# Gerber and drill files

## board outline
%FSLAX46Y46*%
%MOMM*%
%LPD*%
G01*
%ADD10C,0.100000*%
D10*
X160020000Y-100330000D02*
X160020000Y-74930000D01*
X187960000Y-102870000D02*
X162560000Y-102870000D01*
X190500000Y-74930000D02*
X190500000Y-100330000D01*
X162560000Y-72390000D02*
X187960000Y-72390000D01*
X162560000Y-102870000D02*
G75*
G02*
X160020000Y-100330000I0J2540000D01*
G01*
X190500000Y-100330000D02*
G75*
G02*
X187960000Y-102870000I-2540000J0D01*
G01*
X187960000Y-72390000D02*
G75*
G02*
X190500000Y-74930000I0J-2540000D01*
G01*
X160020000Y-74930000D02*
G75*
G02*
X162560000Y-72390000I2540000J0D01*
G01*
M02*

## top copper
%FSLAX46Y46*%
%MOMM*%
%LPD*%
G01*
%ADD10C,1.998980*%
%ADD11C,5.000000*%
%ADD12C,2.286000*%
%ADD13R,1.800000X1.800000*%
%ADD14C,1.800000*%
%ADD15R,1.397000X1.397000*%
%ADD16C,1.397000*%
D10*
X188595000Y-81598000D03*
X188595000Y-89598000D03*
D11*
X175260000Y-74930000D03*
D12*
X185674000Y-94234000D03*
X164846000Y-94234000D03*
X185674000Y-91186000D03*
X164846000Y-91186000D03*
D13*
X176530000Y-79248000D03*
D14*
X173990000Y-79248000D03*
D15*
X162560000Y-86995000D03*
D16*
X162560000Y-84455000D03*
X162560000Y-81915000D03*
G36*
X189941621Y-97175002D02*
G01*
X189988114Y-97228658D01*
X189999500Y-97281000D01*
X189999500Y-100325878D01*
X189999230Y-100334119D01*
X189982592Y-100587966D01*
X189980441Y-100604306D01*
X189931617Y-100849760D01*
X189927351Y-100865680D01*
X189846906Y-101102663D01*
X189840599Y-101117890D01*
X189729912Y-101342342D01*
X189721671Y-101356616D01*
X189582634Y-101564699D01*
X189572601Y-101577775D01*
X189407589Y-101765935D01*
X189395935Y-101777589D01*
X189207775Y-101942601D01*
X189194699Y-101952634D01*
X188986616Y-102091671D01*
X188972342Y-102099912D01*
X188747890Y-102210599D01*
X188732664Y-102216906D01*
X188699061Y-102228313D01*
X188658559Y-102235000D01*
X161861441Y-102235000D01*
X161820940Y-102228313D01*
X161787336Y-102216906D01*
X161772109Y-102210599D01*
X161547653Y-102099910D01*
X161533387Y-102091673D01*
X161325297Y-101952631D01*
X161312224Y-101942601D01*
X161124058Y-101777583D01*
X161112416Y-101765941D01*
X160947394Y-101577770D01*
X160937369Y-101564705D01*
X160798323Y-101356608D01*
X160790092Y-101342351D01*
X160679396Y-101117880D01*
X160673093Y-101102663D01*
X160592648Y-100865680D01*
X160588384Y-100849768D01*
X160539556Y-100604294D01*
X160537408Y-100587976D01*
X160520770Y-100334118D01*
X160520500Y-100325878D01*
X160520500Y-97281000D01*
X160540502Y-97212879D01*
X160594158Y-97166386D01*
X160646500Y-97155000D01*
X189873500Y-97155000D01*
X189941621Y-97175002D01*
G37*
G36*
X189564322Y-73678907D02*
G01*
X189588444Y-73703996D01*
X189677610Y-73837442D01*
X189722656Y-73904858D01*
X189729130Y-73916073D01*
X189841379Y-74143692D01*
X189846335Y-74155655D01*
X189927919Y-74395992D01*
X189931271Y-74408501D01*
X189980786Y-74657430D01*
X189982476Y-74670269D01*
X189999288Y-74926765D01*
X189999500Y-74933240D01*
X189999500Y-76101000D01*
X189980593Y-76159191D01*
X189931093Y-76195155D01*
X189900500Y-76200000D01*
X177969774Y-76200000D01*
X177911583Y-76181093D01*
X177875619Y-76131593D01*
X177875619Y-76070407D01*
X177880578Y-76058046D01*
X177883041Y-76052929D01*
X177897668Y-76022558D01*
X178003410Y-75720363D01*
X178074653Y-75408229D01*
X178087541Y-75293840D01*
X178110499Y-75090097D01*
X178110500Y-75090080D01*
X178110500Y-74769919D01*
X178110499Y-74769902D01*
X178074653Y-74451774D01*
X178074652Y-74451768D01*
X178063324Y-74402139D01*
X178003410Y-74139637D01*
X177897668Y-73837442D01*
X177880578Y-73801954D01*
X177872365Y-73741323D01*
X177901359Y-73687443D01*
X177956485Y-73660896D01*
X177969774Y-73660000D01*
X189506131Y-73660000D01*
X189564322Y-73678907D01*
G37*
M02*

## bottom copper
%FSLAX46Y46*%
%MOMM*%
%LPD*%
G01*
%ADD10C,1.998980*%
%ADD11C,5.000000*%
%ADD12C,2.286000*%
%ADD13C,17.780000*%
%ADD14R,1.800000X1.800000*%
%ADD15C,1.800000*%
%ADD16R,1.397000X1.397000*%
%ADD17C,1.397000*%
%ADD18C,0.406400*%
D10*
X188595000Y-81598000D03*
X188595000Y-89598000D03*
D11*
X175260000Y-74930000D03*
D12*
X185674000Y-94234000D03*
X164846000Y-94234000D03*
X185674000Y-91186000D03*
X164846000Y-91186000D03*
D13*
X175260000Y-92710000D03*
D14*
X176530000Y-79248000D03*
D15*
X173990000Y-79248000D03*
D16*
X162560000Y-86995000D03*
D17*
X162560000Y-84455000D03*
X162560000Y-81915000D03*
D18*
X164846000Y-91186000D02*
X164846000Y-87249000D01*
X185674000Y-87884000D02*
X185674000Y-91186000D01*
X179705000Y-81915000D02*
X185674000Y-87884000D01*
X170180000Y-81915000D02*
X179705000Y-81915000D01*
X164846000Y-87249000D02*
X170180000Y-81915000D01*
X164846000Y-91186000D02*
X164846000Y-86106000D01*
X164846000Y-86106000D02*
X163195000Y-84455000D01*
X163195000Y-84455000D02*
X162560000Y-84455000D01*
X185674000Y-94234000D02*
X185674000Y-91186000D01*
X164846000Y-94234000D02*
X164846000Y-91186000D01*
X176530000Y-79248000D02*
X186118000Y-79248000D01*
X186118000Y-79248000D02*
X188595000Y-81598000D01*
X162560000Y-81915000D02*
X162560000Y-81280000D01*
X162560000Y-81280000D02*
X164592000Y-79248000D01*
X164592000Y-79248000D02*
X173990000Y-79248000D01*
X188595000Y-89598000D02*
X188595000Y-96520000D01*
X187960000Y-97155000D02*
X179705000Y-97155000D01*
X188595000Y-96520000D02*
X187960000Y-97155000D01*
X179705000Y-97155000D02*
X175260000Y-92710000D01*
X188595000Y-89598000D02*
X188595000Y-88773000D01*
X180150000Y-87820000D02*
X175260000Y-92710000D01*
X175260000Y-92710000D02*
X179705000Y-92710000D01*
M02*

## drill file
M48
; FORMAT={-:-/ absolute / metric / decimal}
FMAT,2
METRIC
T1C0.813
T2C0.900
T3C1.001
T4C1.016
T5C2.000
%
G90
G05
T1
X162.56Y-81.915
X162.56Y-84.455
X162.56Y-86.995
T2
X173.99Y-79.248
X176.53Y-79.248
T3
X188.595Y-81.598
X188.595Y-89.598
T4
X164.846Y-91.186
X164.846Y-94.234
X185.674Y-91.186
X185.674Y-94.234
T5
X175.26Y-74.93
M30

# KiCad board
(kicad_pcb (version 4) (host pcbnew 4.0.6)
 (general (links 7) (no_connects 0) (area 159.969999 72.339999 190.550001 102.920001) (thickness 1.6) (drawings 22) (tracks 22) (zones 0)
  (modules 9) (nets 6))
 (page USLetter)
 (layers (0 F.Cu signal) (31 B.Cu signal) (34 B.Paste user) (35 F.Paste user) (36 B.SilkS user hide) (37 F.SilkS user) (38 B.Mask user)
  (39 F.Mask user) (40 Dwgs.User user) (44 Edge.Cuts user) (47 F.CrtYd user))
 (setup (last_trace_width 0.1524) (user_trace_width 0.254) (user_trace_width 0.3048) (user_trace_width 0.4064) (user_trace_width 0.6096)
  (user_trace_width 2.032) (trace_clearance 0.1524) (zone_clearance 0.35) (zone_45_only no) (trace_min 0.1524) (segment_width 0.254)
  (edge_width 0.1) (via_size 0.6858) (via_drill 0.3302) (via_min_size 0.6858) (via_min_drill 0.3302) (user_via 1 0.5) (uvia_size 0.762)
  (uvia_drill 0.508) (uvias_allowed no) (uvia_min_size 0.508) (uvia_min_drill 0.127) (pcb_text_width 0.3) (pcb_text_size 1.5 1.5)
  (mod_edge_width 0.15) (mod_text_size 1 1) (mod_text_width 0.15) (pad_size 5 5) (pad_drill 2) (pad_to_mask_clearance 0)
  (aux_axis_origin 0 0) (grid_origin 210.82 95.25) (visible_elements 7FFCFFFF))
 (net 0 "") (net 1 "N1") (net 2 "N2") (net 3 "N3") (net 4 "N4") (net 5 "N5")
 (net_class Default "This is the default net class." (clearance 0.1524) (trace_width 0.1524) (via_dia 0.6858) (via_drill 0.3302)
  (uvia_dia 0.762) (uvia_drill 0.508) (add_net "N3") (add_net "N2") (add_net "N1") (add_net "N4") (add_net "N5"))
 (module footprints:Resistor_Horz (layer F.Cu) (at 188.595 85.598 270)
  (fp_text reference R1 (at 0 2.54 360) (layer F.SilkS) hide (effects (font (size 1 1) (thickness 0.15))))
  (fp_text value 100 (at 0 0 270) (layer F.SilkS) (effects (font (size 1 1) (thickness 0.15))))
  (pad 1 thru_hole circle (at -4 0 270) (size 1.99898 1.99898) (drill 1.00076) (layers *.Cu *.SilkS *.Mask) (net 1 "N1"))
  (pad 2 thru_hole circle (at 4 0 270) (size 1.99898 1.99898) (drill 1.00076) (layers *.Cu *.SilkS *.Mask) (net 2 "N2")))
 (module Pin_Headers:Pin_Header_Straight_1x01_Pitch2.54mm (layer F.Cu) (at 175.26 74.93)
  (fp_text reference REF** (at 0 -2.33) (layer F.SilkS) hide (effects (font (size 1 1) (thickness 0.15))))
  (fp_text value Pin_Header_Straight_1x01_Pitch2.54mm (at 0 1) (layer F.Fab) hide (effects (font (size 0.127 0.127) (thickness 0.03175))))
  (pad 1 thru_hole circle (at 0 0) (size 5 5) (drill 2) (layers *.Cu B.Mask)))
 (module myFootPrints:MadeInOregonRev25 (layer F.Cu) (at 167.64 76.454)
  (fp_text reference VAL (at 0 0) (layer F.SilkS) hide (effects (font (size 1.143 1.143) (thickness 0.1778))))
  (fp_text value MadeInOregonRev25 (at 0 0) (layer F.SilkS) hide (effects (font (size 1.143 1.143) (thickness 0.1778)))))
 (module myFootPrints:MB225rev (layer F.Cu) (at 184.15 76.2)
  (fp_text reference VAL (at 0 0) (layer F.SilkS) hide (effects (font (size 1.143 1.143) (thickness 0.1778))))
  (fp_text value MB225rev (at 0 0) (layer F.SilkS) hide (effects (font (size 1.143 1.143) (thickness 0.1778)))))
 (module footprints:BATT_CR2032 (layer B.Cu) (at 175.26 92.71 180)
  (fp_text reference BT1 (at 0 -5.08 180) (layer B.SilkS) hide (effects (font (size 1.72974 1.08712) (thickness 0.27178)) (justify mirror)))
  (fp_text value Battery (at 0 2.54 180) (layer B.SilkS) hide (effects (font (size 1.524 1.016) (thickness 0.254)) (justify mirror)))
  (pad 1 thru_hole circle (at -10.414 -1.524 180) (size 2.286 2.286) (drill 1.016) (layers *.Cu *.Mask B.SilkS) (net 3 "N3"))
  (pad 1 thru_hole circle (at 10.414 -1.524 180) (size 2.286 2.286) (drill 1.016) (layers *.Cu *.Mask B.SilkS) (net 3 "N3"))
  (pad 1 thru_hole circle (at -10.414 1.524 180) (size 2.286 2.286) (drill 1.016) (layers *.Cu *.Mask B.SilkS) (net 3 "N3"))
  (pad 1 thru_hole circle (at 10.414 1.524 180) (size 2.286 2.286) (drill 1.016) (layers *.Cu *.Mask B.SilkS) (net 3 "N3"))
  (pad 2 smd circle (at 0 0 180) (size 17.78 17.78) (layers B.Cu B.Paste B.Mask) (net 2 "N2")))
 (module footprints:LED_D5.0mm (layer F.Cu) (at 176.53 79.248 180)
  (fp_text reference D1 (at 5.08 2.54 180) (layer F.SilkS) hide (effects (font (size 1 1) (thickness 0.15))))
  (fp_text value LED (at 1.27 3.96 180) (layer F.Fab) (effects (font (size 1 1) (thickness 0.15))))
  (pad 1 thru_hole rect (at 0 0 180) (size 1.8 1.8) (drill 0.9) (layers *.Cu *.Mask) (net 1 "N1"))
  (pad 2 thru_hole circle (at 2.54 0 180) (size 1.8 1.8) (drill 0.9) (layers *.Cu *.Mask) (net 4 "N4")))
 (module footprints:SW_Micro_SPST (layer F.Cu) (at 162.56 84.455 90)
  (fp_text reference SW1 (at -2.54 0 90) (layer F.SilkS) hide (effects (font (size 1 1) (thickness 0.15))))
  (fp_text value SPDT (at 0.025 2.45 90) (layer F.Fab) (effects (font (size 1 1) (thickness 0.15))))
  (pad 1 thru_hole rect (at -2.54 0 90) (size 1.397 1.397) (drill 0.8128) (layers *.Cu *.Mask F.SilkS) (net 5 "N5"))
  (pad 2 thru_hole circle (at 0 0 90) (size 1.397 1.397) (drill 0.8128) (layers *.Cu *.Mask F.SilkS) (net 3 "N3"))
  (pad 3 thru_hole circle (at 2.54 0 90) (size 1.397 1.397) (drill 0.8128) (layers *.Cu *.Mask F.SilkS) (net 4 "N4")))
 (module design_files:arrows (layer F.Cu) (at 179.07 77.47)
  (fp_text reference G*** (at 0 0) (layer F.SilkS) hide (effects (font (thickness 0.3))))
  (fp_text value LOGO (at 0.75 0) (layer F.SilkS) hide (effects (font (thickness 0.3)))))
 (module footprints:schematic (layer F.Cu) (at 175.26 87.503)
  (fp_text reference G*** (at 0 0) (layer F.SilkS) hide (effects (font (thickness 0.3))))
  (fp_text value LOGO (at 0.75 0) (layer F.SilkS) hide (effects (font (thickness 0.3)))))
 (gr_line (start 160.02 100.33) (end 160.02 74.93) (angle 90) (layer Edge.Cuts) (width 0.1))
 (gr_line (start 187.96 102.87) (end 162.56 102.87) (angle 90) (layer Edge.Cuts) (width 0.1))
 (gr_line (start 190.5 74.93) (end 190.5 100.33) (angle 90) (layer Edge.Cuts) (width 0.1))
 (gr_line (start 162.56 72.39) (end 187.96 72.39) (angle 90) (layer Edge.Cuts) (width 0.1))
 (gr_arc (start 162.56 100.33) (end 162.56 102.87) (angle 90) (layer Edge.Cuts) (width 0.1))
 (gr_arc (start 187.96 100.33) (end 190.5 100.33) (angle 90) (layer Edge.Cuts) (width 0.1))
 (gr_arc (start 187.96 74.93) (end 187.96 72.39) (angle 90) (layer Edge.Cuts) (width 0.1))
 (gr_arc (start 162.56 74.93) (end 160.02 74.93) (angle 90) (layer Edge.Cuts) (width 0.1))
 (segment (start 164.846 91.186) (end 164.846 87.249) (width 0.4064) (layer B.Cu) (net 3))
 (segment (start 185.674 87.884) (end 185.674 91.186) (width 0.4064) (layer B.Cu) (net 3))
 (segment (start 179.705 81.915) (end 185.674 87.884) (width 0.4064) (layer B.Cu) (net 3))
 (segment (start 170.18 81.915) (end 179.705 81.915) (width 0.4064) (layer B.Cu) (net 3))
 (segment (start 164.846 87.249) (end 170.18 81.915) (width 0.4064) (layer B.Cu) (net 3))
 (segment (start 164.846 91.186) (end 164.846 86.106) (width 0.4064) (layer B.Cu) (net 3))
 (segment (start 164.846 86.106) (end 163.195 84.455) (width 0.4064) (layer B.Cu) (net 3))
 (segment (start 163.195 84.455) (end 162.56 84.455) (width 0.4064) (layer B.Cu) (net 3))
 (segment (start 185.674 94.234) (end 185.674 91.186) (width 0.4064) (layer B.Cu) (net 3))
 (segment (start 164.846 94.234) (end 164.846 91.186) (width 0.4064) (layer B.Cu) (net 3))
 (segment (start 176.53 79.248) (end 186.118 79.248) (width 0.4064) (layer B.Cu) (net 1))
 (segment (start 186.118 79.248) (end 188.595 81.598) (width 0.4064) (layer B.Cu) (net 1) (status 20))
 (segment (start 162.56 81.915) (end 162.56 81.28) (width 0.4064) (layer B.Cu) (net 4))
 (segment (start 162.56 81.28) (end 164.592 79.248) (width 0.4064) (layer B.Cu) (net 4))
 (segment (start 164.592 79.248) (end 173.99 79.248) (width 0.4064) (layer B.Cu) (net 4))
 (segment (start 188.595 89.598) (end 188.595 96.52) (width 0.4064) (layer B.Cu) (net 2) (status 10))
 (segment (start 187.96 97.155) (end 179.705 97.155) (width 0.4064) (layer B.Cu) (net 2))
 (segment (start 188.595 96.52) (end 187.96 97.155) (width 0.4064) (layer B.Cu) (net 2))
 (segment (start 179.705 97.155) (end 175.26 92.71) (width 0.4064) (layer B.Cu) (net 2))
 (segment (start 188.595 89.598) (end 188.595 88.773) (width 0.4064) (layer B.Cu) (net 2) (status 30))
 (segment (start 180.15 87.82) (end 175.26 92.71) (width 0.4064) (layer B.Cu) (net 2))
 (segment (start 175.26 92.71) (end 179.705 92.71) (width 0.4064) (layer B.Cu) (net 2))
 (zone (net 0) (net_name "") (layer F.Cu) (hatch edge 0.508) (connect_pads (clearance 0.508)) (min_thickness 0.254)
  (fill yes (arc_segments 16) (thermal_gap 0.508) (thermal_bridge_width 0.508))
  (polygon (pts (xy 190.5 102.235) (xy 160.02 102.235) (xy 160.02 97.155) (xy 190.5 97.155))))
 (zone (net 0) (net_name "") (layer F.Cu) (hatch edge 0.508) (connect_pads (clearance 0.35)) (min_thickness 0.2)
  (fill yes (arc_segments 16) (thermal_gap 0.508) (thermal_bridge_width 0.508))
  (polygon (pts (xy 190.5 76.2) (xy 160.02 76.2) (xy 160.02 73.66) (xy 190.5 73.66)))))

